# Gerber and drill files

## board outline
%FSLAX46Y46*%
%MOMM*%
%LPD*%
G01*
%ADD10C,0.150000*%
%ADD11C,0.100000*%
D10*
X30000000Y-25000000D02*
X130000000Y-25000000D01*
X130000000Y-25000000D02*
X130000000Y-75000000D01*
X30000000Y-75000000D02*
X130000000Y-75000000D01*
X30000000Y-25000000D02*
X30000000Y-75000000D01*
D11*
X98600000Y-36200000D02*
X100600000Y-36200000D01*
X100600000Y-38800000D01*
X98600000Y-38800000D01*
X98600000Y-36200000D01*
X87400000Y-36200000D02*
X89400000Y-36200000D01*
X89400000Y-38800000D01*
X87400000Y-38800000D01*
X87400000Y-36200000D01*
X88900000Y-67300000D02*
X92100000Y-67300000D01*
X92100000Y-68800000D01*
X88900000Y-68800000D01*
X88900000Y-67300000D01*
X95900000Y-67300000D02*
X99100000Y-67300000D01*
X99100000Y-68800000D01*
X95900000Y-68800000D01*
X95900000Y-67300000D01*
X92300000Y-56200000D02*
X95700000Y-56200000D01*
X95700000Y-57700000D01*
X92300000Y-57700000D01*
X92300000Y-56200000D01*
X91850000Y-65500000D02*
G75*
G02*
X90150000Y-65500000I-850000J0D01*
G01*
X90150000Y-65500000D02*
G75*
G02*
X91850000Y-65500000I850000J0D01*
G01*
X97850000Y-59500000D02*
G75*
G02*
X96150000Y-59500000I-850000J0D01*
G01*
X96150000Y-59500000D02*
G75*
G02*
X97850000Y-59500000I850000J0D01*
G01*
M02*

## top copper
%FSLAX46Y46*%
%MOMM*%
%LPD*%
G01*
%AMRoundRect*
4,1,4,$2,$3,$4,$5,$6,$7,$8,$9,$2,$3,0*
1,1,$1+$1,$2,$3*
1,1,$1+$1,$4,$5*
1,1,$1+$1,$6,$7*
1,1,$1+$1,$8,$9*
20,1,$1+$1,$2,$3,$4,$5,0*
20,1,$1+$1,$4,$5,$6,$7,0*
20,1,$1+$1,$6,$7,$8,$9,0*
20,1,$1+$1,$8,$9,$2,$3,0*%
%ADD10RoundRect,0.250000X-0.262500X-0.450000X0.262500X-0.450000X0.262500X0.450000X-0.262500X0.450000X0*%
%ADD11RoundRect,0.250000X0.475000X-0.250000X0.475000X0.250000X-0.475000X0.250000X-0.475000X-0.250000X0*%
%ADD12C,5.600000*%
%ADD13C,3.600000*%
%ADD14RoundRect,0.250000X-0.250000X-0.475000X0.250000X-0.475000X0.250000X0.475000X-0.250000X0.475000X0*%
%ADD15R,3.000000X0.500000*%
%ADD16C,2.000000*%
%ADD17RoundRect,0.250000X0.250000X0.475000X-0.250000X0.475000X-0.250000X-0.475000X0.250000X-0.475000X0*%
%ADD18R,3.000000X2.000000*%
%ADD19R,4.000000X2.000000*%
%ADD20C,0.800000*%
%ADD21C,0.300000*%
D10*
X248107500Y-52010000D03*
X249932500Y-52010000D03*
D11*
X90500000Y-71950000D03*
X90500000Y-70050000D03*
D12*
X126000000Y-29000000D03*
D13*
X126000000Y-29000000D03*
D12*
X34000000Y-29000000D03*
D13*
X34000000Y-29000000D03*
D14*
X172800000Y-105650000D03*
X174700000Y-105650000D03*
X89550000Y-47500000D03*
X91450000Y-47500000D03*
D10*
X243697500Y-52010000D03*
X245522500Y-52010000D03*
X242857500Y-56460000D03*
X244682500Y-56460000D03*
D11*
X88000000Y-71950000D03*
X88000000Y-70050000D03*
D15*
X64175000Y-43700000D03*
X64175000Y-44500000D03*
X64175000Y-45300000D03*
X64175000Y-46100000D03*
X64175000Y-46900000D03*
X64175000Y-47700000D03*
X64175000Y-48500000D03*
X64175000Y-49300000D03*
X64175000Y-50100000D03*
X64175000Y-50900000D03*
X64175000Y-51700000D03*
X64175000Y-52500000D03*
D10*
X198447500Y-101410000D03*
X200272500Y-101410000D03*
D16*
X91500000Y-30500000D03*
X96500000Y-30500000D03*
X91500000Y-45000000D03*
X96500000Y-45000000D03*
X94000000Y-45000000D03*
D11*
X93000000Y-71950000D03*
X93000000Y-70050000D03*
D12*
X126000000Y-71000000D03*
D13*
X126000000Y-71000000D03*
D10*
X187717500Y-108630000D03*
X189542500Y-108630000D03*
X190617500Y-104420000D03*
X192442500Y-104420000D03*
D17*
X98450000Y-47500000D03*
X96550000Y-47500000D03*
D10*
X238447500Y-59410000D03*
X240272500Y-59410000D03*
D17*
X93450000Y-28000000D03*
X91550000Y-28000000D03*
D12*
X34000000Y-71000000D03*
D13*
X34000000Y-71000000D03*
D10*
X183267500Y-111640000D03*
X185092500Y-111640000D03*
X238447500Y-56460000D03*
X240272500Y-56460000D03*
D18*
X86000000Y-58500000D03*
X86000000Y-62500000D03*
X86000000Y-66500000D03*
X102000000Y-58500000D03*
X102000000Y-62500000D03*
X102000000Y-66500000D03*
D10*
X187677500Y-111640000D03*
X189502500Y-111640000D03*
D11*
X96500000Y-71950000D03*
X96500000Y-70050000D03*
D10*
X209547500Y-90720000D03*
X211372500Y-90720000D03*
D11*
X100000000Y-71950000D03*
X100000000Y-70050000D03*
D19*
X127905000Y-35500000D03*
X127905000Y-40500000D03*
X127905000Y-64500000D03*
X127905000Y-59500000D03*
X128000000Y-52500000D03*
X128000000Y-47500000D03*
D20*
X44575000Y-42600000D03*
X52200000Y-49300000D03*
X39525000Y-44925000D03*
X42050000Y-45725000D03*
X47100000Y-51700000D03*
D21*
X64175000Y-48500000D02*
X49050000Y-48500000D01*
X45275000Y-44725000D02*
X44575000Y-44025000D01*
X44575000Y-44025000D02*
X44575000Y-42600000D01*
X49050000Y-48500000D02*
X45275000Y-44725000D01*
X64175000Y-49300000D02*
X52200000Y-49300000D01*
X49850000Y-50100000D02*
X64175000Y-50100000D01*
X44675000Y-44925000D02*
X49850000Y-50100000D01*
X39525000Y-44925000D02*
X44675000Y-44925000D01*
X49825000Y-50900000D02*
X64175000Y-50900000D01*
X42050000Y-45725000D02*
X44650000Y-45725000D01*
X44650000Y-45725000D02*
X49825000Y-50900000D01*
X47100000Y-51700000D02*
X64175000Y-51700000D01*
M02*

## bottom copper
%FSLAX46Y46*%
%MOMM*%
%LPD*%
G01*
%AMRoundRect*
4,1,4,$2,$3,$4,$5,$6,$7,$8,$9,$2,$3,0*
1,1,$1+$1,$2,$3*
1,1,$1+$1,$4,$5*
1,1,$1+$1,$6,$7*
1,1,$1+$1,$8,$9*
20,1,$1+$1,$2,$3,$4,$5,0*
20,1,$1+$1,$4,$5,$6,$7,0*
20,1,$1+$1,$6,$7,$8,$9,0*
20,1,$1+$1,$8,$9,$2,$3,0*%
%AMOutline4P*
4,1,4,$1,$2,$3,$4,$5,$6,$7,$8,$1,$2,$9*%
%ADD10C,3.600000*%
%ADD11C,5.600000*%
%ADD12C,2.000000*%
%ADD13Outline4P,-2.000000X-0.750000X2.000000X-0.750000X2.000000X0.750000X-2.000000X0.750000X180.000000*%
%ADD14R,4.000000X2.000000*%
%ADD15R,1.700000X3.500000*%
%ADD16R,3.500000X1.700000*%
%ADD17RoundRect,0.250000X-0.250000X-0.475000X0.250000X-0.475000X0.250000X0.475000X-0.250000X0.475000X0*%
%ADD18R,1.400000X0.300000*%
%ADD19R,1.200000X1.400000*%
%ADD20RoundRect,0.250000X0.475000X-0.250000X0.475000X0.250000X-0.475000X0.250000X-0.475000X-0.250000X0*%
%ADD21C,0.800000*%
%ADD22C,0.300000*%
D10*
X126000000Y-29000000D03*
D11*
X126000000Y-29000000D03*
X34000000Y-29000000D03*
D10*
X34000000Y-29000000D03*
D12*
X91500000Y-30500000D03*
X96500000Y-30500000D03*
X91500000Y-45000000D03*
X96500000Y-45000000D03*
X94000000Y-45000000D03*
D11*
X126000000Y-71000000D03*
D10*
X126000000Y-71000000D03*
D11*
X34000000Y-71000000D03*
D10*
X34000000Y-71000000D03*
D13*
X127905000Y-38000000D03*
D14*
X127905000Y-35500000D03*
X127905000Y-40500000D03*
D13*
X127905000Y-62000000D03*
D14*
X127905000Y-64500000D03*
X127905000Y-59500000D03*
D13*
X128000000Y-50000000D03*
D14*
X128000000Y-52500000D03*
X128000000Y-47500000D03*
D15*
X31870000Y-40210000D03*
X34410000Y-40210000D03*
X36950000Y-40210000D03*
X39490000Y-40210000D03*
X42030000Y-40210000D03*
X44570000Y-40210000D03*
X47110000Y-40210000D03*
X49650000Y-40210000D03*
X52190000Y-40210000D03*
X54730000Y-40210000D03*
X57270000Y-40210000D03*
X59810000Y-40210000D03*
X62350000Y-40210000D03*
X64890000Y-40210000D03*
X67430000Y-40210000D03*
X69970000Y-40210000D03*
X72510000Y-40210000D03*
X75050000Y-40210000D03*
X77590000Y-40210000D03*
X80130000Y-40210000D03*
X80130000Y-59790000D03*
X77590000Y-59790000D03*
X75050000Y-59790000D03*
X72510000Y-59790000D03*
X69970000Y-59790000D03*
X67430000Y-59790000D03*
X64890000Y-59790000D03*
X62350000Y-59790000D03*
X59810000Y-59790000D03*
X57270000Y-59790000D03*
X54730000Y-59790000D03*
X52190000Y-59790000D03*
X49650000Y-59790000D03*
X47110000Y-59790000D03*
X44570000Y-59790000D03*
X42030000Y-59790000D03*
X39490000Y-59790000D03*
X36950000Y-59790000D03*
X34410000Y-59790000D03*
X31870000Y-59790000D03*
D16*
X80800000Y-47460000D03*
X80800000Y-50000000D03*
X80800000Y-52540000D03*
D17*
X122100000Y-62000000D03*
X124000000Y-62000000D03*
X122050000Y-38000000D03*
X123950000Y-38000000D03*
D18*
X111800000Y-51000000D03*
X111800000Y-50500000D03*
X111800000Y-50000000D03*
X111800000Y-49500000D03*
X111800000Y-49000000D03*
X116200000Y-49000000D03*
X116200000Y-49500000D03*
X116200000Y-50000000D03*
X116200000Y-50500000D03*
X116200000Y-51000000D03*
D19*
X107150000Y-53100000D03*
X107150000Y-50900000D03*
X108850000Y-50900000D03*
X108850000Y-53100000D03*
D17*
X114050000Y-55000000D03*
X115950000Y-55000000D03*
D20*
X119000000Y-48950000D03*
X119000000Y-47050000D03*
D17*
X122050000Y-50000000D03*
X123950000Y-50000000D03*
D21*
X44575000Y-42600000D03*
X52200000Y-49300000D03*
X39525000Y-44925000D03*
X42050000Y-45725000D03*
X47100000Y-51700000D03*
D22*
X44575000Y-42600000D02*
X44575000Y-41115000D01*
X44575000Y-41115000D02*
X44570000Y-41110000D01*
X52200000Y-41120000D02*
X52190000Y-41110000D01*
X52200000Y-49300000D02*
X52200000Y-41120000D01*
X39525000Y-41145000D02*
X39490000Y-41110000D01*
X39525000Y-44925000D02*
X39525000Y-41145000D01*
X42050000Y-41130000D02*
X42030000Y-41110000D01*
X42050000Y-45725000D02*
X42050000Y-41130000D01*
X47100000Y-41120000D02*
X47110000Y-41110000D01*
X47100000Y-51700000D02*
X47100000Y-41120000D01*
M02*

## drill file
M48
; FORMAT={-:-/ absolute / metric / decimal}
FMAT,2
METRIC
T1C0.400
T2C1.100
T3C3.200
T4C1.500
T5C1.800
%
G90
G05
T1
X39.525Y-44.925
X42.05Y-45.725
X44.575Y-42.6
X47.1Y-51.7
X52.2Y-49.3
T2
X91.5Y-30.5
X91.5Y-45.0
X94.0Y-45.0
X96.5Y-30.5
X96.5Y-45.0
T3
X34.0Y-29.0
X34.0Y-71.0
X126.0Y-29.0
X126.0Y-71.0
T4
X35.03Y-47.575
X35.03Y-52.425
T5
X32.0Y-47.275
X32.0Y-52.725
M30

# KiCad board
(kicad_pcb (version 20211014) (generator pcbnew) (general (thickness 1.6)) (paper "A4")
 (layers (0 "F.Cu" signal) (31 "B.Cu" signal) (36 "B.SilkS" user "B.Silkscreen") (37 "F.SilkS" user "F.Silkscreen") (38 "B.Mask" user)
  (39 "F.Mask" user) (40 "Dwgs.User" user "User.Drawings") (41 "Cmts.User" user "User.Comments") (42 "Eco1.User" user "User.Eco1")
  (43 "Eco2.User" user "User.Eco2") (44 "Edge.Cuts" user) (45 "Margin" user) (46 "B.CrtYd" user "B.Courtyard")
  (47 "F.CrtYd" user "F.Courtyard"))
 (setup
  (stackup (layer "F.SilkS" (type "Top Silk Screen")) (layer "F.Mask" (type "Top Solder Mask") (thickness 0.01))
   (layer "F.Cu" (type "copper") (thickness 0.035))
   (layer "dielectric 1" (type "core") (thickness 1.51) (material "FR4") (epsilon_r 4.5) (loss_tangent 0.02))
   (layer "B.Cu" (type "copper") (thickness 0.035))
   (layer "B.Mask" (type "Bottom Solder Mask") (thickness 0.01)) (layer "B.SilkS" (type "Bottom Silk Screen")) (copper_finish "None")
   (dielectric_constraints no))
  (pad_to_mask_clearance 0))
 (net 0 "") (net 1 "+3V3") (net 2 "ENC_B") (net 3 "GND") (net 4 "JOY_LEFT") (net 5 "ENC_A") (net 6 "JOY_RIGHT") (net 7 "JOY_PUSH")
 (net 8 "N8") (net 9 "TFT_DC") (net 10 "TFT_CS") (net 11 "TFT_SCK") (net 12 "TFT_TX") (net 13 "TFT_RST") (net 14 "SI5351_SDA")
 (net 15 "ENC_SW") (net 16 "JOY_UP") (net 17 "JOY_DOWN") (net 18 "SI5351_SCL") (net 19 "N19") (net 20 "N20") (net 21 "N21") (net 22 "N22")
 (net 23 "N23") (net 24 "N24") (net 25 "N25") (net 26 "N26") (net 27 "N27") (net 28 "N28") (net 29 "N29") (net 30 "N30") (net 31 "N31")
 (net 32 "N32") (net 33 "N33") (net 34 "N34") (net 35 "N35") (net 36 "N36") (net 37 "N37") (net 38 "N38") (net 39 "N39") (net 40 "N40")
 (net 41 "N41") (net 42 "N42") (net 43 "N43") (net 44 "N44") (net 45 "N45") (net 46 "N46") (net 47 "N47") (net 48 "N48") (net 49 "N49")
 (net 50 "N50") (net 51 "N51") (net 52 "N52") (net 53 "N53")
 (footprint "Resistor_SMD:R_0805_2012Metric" (layer "F.Cu") (at 249.02 52.01)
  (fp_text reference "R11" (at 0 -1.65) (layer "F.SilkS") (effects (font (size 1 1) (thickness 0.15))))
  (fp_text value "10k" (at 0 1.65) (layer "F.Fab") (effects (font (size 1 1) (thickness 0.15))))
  (pad "1" smd roundrect (at -0.9125 0) (size 1.025 1.4) (layers "F.Cu" "F.Paste" "F.Mask") (roundrect_rratio 0.243902) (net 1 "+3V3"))
  (pad "2" smd roundrect (at 0.9125 0) (size 1.025 1.4) (layers "F.Cu" "F.Paste" "F.Mask") (roundrect_rratio 0.243902) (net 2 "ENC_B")))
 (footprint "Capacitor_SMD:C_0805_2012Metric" (layer "F.Cu") (at 90.5 71 90)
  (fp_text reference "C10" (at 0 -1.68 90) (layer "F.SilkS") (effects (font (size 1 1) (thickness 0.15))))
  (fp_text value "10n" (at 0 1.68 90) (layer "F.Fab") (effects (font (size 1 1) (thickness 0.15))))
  (pad "1" smd roundrect (at -0.95 0 90) (size 1 1.45) (layers "F.Cu" "F.Paste" "F.Mask") (roundrect_rratio 0.25) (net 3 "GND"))
  (pad "2" smd roundrect (at 0.95 0 90) (size 1 1.45) (layers "F.Cu" "F.Paste" "F.Mask") (roundrect_rratio 0.25) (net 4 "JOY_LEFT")))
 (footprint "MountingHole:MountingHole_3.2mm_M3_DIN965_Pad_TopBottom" (layer "F.Cu") (at 126 29)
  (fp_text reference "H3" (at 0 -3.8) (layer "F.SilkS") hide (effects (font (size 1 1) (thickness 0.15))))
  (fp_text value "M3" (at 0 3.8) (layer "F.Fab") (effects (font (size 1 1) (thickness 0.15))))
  (pad "1" connect circle (at 0 0) (size 5.6 5.6) (layers "F.Cu" "F.Mask"))
  (pad "1" thru_hole circle (at 0 0) (size 3.6 3.6) (drill 3.2) (layers *.Cu *.Mask))
  (pad "1" connect circle (at 0 0) (size 5.6 5.6) (layers "B.Cu" "B.Mask")))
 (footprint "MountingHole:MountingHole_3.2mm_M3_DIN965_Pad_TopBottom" (layer "F.Cu") (at 34 29)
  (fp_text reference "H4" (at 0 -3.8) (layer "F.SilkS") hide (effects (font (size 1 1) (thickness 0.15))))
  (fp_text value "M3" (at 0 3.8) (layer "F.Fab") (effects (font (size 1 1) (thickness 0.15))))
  (pad "1" connect circle (at 0 0) (size 5.6 5.6) (layers "F.Cu" "F.Mask"))
  (pad "1" connect circle (at 0 0) (size 5.6 5.6) (layers "B.Cu" "B.Mask"))
  (pad "1" thru_hole circle (at 0 0) (size 3.6 3.6) (drill 3.2) (layers *.Cu *.Mask)))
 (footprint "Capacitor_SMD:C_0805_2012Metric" (layer "F.Cu") (at 173.75 105.65)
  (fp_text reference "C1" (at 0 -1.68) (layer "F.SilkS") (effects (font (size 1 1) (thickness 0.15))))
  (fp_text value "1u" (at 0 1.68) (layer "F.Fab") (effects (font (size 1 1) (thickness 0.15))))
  (pad "1" smd roundrect (at -0.95 0) (size 1 1.45) (layers "F.Cu" "F.Paste" "F.Mask") (roundrect_rratio 0.25) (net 1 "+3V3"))
  (pad "2" smd roundrect (at 0.95 0) (size 1 1.45) (layers "F.Cu" "F.Paste" "F.Mask") (roundrect_rratio 0.25) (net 3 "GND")))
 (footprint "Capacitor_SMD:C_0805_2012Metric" (layer "F.Cu") (at 90.5 47.5)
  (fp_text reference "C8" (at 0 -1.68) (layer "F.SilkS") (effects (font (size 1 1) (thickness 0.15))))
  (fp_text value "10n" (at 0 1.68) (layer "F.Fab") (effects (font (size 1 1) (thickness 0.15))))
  (pad "1" smd roundrect (at -0.95 0) (size 1 1.45) (layers "F.Cu" "F.Paste" "F.Mask") (roundrect_rratio 0.25) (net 3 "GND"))
  (pad "2" smd roundrect (at 0.95 0) (size 1 1.45) (layers "F.Cu" "F.Paste" "F.Mask") (roundrect_rratio 0.25) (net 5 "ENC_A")))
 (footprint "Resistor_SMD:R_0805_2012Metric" (layer "F.Cu") (at 244.61 52.01)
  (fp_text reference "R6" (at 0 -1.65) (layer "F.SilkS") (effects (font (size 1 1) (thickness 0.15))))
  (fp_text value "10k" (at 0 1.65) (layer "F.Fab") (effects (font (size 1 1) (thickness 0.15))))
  (pad "1" smd roundrect (at -0.9125 0) (size 1.025 1.4) (layers "F.Cu" "F.Paste" "F.Mask") (roundrect_rratio 0.243902) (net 1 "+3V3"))
  (pad "2" smd roundrect (at 0.9125 0) (size 1.025 1.4) (layers "F.Cu" "F.Paste" "F.Mask") (roundrect_rratio 0.243902) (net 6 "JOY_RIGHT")))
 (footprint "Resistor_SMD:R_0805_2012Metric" (layer "F.Cu") (at 243.77 56.46)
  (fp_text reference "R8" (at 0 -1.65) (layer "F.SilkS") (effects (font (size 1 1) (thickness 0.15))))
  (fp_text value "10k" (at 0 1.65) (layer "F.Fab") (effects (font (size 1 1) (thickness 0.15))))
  (pad "1" smd roundrect (at -0.9125 0) (size 1.025 1.4) (layers "F.Cu" "F.Paste" "F.Mask") (roundrect_rratio 0.243902) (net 1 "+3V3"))
  (pad "2" smd roundrect (at 0.9125 0) (size 1.025 1.4) (layers "F.Cu" "F.Paste" "F.Mask") (roundrect_rratio 0.243902) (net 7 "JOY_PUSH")))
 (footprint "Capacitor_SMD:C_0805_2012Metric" (layer "F.Cu") (at 88 71 90)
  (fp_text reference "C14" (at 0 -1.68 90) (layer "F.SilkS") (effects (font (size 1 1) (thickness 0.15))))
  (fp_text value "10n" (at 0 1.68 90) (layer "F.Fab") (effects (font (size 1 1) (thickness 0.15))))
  (pad "1" smd roundrect (at -0.95 0 90) (size 1 1.45) (layers "F.Cu" "F.Paste" "F.Mask") (roundrect_rratio 0.25) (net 3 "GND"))
  (pad "2" smd roundrect (at 0.95 0 90) (size 1 1.45) (layers "F.Cu" "F.Paste" "F.Mask") (roundrect_rratio 0.25) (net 7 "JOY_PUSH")))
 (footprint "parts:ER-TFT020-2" (layer "F.Cu") (at 58 50)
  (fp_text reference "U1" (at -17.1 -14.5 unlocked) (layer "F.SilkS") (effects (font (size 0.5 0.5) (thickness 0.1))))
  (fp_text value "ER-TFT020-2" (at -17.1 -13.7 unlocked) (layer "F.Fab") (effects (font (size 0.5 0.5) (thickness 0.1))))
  (pad "1" smd rect (at 6.175 -6.3) (size 3 0.5) (layers "F.Cu" "B.Paste" "B.Mask") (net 3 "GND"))
  (pad "2" smd rect (at 6.175 -5.5) (size 3 0.5) (layers "F.Cu" "B.Paste" "B.Mask") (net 3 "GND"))
  (pad "3" smd rect (at 6.175 -4.7) (size 3 0.5) (layers "F.Cu" "B.Paste" "B.Mask") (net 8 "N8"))
  (pad "4" smd rect (at 6.175 -3.9) (size 3 0.5) (layers "F.Cu" "B.Paste" "B.Mask") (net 1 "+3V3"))
  (pad "5" smd rect (at 6.175 -3.1) (size 3 0.5) (layers "F.Cu" "B.Paste" "B.Mask") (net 3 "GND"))
  (pad "6" smd rect (at 6.175 -2.3) (size 3 0.5) (layers "F.Cu" "B.Paste" "B.Mask") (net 3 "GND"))
  (pad "7" smd rect (at 6.175 -1.5) (size 3 0.5) (layers "F.Cu" "B.Paste" "B.Mask") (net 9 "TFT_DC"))
  (pad "8" smd rect (at 6.175 -0.7) (size 3 0.5) (layers "F.Cu" "B.Paste" "B.Mask") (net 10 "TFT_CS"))
  (pad "9" smd rect (at 6.175 0.1) (size 3 0.5) (layers "F.Cu" "B.Paste" "B.Mask") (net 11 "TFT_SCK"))
  (pad "10" smd rect (at 6.175 0.9) (size 3 0.5) (layers "F.Cu" "B.Paste" "B.Mask") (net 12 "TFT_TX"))
  (pad "11" smd rect (at 6.175 1.7) (size 3 0.5) (layers "F.Cu" "B.Paste" "B.Mask") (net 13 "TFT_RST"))
  (pad "12" smd rect (at 6.175 2.5) (size 3 0.5) (layers "F.Cu" "B.Paste" "B.Mask") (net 3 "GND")))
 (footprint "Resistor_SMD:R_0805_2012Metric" (layer "F.Cu") (at 199.36 101.41)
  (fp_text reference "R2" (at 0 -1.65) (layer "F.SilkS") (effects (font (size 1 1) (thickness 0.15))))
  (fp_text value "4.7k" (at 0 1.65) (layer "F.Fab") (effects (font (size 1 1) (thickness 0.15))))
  (pad "1" smd roundrect (at -0.9125 0) (size 1.025 1.4) (layers "F.Cu" "F.Paste" "F.Mask") (roundrect_rratio 0.243902)
   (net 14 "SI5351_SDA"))
  (pad "2" smd roundrect (at 0.9125 0) (size 1.025 1.4) (layers "F.Cu" "F.Paste" "F.Mask") (roundrect_rratio 0.243902) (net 1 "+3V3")))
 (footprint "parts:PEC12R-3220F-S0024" (layer "F.Cu") (at 94 37.5)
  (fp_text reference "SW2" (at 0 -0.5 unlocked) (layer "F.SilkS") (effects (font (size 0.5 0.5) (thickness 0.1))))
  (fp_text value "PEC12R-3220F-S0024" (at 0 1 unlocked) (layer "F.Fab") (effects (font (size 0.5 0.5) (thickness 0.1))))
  (fp_rect (start 4.6 -1.3) (end 6.6 1.3) (layer "Edge.Cuts") (width 0.1) (fill none))
  (fp_rect (start -6.6 -1.3) (end -4.6 1.3) (layer "Edge.Cuts") (width 0.1) (fill none))
  (pad "1" thru_hole circle (at -2.5 -7) (size 2 2) (drill 1.1) (layers *.Cu *.Mask) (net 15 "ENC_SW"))
  (pad "2" thru_hole circle (at 2.5 -7) (size 2 2) (drill 1.1) (layers *.Cu *.Mask) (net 3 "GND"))
  (pad "A" thru_hole circle (at -2.5 7.5) (size 2 2) (drill 1.1) (layers *.Cu *.Mask) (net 5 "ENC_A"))
  (pad "B" thru_hole circle (at 2.5 7.5) (size 2 2) (drill 1.1) (layers *.Cu *.Mask) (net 2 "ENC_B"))
  (pad "C" thru_hole circle (at 0 7.5) (size 2 2) (drill 1.1) (layers *.Cu *.Mask) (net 3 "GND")))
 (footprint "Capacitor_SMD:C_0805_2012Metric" (layer "F.Cu") (at 93 71 90)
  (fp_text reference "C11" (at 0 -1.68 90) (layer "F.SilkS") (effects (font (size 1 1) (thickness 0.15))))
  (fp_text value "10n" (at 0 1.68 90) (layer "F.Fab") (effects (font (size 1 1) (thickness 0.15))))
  (pad "1" smd roundrect (at -0.95 0 90) (size 1 1.45) (layers "F.Cu" "F.Paste" "F.Mask") (roundrect_rratio 0.25) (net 3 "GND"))
  (pad "2" smd roundrect (at 0.95 0 90) (size 1 1.45) (layers "F.Cu" "F.Paste" "F.Mask") (roundrect_rratio 0.25) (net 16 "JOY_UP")))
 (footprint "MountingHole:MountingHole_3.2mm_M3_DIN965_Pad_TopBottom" (layer "F.Cu") (at 126 71)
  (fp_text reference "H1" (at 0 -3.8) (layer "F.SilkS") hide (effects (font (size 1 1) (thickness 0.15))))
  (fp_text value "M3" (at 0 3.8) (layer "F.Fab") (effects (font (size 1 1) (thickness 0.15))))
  (pad "1" connect circle (at 0 0) (size 5.6 5.6) (layers "B.Cu" "B.Mask"))
  (pad "1" connect circle (at 0 0) (size 5.6 5.6) (layers "F.Cu" "F.Mask"))
  (pad "1" thru_hole circle (at 0 0) (size 3.6 3.6) (drill 3.2) (layers *.Cu *.Mask)))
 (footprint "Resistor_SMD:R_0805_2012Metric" (layer "F.Cu") (at 188.63 108.63)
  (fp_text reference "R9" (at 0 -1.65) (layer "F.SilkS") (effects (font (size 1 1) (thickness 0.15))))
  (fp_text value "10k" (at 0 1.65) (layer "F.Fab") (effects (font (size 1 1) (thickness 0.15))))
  (pad "1" smd roundrect (at -0.9125 0) (size 1.025 1.4) (layers "F.Cu" "F.Paste" "F.Mask") (roundrect_rratio 0.243902) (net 1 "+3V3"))
  (pad "2" smd roundrect (at 0.9125 0) (size 1.025 1.4) (layers "F.Cu" "F.Paste" "F.Mask") (roundrect_rratio 0.243902) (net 15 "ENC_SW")))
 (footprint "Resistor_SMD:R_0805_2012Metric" (layer "F.Cu") (at 191.53 104.42)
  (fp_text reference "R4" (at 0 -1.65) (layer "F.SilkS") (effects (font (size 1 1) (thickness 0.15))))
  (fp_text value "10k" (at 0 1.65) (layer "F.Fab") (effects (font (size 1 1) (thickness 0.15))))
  (pad "1" smd roundrect (at -0.9125 0) (size 1.025 1.4) (layers "F.Cu" "F.Paste" "F.Mask") (roundrect_rratio 0.243902) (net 1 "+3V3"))
  (pad "2" smd roundrect (at 0.9125 0) (size 1.025 1.4) (layers "F.Cu" "F.Paste" "F.Mask") (roundrect_rratio 0.243902) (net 4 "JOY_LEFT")))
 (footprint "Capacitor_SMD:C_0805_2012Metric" (layer "F.Cu") (at 97.5 47.5 180)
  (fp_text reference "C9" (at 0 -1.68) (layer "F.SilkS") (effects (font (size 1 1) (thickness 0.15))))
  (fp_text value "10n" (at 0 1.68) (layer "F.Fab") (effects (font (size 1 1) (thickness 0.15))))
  (pad "1" smd roundrect (at -0.95 0 180) (size 1 1.45) (layers "F.Cu" "F.Paste" "F.Mask") (roundrect_rratio 0.25) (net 3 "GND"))
  (pad "2" smd roundrect (at 0.95 0 180) (size 1 1.45) (layers "F.Cu" "F.Paste" "F.Mask") (roundrect_rratio 0.25) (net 2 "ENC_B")))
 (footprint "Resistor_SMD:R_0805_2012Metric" (layer "F.Cu") (at 239.36 59.41)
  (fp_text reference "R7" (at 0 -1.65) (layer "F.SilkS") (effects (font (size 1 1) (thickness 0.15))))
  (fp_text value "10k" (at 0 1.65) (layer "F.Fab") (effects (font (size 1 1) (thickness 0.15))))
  (pad "1" smd roundrect (at -0.9125 0) (size 1.025 1.4) (layers "F.Cu" "F.Paste" "F.Mask") (roundrect_rratio 0.243902) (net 1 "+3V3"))
  (pad "2" smd roundrect (at 0.9125 0) (size 1.025 1.4) (layers "F.Cu" "F.Paste" "F.Mask") (roundrect_rratio 0.243902) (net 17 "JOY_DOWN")))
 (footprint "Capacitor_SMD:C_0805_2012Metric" (layer "F.Cu") (at 92.5 28 180)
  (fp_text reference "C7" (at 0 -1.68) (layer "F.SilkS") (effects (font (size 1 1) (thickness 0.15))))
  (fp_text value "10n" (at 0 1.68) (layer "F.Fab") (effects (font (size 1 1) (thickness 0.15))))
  (pad "1" smd roundrect (at -0.95 0 180) (size 1 1.45) (layers "F.Cu" "F.Paste" "F.Mask") (roundrect_rratio 0.25) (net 3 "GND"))
  (pad "2" smd roundrect (at 0.95 0 180) (size 1 1.45) (layers "F.Cu" "F.Paste" "F.Mask") (roundrect_rratio 0.25) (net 15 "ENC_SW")))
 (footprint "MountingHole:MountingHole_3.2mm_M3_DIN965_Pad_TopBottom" (layer "F.Cu") (at 34 71)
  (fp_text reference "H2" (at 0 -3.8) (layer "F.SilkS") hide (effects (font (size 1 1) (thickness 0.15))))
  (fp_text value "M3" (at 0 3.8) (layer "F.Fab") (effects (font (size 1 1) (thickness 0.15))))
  (pad "1" connect circle (at 0 0) (size 5.6 5.6) (layers "B.Cu" "B.Mask"))
  (pad "1" connect circle (at 0 0) (size 5.6 5.6) (layers "F.Cu" "F.Mask"))
  (pad "1" thru_hole circle (at 0 0) (size 3.6 3.6) (drill 3.2) (layers *.Cu *.Mask)))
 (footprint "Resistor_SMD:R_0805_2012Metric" (layer "F.Cu") (at 184.18 111.64)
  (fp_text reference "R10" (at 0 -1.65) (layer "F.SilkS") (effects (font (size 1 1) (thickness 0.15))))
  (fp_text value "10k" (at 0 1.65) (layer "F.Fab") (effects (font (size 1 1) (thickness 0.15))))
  (pad "1" smd roundrect (at -0.9125 0) (size 1.025 1.4) (layers "F.Cu" "F.Paste" "F.Mask") (roundrect_rratio 0.243902) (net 1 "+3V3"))
  (pad "2" smd roundrect (at 0.9125 0) (size 1.025 1.4) (layers "F.Cu" "F.Paste" "F.Mask") (roundrect_rratio 0.243902) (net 5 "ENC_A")))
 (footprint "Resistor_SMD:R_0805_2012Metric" (layer "F.Cu") (at 239.36 56.46)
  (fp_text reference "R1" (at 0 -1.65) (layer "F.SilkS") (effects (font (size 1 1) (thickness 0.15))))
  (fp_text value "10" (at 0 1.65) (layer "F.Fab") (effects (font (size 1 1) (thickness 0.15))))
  (pad "1" smd roundrect (at -0.9125 0) (size 1.025 1.4) (layers "F.Cu" "F.Paste" "F.Mask") (roundrect_rratio 0.243902) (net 8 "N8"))
  (pad "2" smd roundrect (at 0.9125 0) (size 1.025 1.4) (layers "F.Cu" "F.Paste" "F.Mask") (roundrect_rratio 0.243902) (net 1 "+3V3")))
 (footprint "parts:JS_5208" (layer "F.Cu") (at 94 62.5)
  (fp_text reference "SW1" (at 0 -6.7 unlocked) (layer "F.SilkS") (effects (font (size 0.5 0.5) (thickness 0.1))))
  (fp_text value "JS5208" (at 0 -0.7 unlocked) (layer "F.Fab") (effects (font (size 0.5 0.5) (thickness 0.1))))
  (fp_rect (start -5.1 4.8) (end -1.9 6.3) (layer "Edge.Cuts") (width 0.1) (fill none))
  (fp_rect (start 1.9 4.8) (end 5.1 6.3) (layer "Edge.Cuts") (width 0.1) (fill none))
  (fp_rect (start -1.7 -6.3) (end 1.7 -4.8) (layer "Edge.Cuts") (width 0.1) (fill none))
  (fp_circle (center -3 3) (end -2.15 3) (layer "Edge.Cuts") (width 0.1) (fill none))
  (fp_circle (center 3 -3) (end 3.85 -3) (layer "Edge.Cuts") (width 0.1) (fill none))
  (pad "1" smd rect (at -8 -4) (size 3 2) (layers "F.Cu" "F.Paste" "F.Mask") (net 3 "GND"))
  (pad "2" smd rect (at -8 0) (size 3 2) (layers "F.Cu" "F.Paste" "F.Mask") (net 4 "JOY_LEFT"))
  (pad "3" smd rect (at -8 4) (size 3 2) (layers "F.Cu" "F.Paste" "F.Mask") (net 7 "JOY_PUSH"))
  (pad "4" smd rect (at 8 -4) (size 3 2) (layers "F.Cu" "F.Paste" "F.Mask") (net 16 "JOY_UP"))
  (pad "5" smd rect (at 8 0) (size 3 2) (layers "F.Cu" "F.Paste" "F.Mask") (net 6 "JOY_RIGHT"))
  (pad "6" smd rect (at 8 4) (size 3 2) (layers "F.Cu" "F.Paste" "F.Mask") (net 17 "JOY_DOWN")))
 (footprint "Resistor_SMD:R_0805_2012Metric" (layer "F.Cu") (at 188.59 111.64)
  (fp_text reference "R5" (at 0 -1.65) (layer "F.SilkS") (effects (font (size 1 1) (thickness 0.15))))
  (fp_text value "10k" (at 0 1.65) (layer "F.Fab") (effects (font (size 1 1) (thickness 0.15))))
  (pad "1" smd roundrect (at -0.9125 0) (size 1.025 1.4) (layers "F.Cu" "F.Paste" "F.Mask") (roundrect_rratio 0.243902) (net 1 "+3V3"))
  (pad "2" smd roundrect (at 0.9125 0) (size 1.025 1.4) (layers "F.Cu" "F.Paste" "F.Mask") (roundrect_rratio 0.243902) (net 16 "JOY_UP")))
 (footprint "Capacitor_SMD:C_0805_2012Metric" (layer "F.Cu") (at 96.5 71 90)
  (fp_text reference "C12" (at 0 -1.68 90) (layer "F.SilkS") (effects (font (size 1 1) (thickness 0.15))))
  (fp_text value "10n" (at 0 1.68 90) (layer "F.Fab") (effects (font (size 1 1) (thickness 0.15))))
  (pad "1" smd roundrect (at -0.95 0 90) (size 1 1.45) (layers "F.Cu" "F.Paste" "F.Mask") (roundrect_rratio 0.25) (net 3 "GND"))
  (pad "2" smd roundrect (at 0.95 0 90) (size 1 1.45) (layers "F.Cu" "F.Paste" "F.Mask") (roundrect_rratio 0.25) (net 6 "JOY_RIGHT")))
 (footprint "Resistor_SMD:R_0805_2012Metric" (layer "F.Cu") (at 210.46 90.72)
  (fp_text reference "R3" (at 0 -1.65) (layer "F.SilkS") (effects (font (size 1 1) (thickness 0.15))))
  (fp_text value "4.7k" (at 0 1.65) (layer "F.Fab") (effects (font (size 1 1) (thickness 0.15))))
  (pad "1" smd roundrect (at -0.9125 0) (size 1.025 1.4) (layers "F.Cu" "F.Paste" "F.Mask") (roundrect_rratio 0.243902)
   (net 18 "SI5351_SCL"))
  (pad "2" smd roundrect (at 0.9125 0) (size 1.025 1.4) (layers "F.Cu" "F.Paste" "F.Mask") (roundrect_rratio 0.243902) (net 1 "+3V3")))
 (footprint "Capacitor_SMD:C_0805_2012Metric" (layer "F.Cu") (at 100 71 90)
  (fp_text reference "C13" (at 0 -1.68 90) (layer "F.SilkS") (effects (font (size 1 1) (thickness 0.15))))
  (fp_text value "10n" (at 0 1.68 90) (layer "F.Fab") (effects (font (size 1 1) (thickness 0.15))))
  (pad "1" smd roundrect (at -0.95 0 90) (size 1 1.45) (layers "F.Cu" "F.Paste" "F.Mask") (roundrect_rratio 0.25) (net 3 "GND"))
  (pad "2" smd roundrect (at 0.95 0 90) (size 1 1.45) (layers "F.Cu" "F.Paste" "F.Mask") (roundrect_rratio 0.25) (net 17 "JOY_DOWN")))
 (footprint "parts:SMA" (layer "B.Cu") (at 129.905 38 180)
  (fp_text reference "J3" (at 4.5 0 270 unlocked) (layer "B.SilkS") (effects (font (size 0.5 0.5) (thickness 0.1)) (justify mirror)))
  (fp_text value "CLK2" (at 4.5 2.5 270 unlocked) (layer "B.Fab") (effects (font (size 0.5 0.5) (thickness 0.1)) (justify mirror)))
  (pad "1" smd trapezoid (at 2 0 180) (size 4 1.5) (layers "B.Cu" "B.Paste" "B.Mask") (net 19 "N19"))
  (pad "2" smd rect (at 2 2.5 180) (size 4 2) (layers "B.Cu" "B.Paste" "B.Mask") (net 3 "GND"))
  (pad "2" smd rect (at 2 2.5 180) (size 4 2) (layers "F.Cu" "B.Paste" "B.Mask") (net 3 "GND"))
  (pad "2" smd rect (at 2 -2.5 180) (size 4 2) (layers "B.Cu" "B.Paste" "B.Mask") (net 3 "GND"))
  (pad "2" smd rect (at 2 -2.5 180) (size 4 2) (layers "F.Cu" "B.Paste" "B.Mask") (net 3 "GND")))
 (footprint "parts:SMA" (layer "B.Cu") (at 129.905 62 180)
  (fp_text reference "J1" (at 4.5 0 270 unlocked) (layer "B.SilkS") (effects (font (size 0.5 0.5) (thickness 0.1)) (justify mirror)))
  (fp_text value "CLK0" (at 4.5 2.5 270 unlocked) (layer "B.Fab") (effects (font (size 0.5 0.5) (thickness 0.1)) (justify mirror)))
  (pad "1" smd trapezoid (at 2 0 180) (size 4 1.5) (layers "B.Cu" "B.Paste" "B.Mask") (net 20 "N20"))
  (pad "2" smd rect (at 2 -2.5 180) (size 4 2) (layers "B.Cu" "B.Paste" "B.Mask") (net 3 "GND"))
  (pad "2" smd rect (at 2 -2.5 180) (size 4 2) (layers "F.Cu" "B.Paste" "B.Mask") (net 3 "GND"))
  (pad "2" smd rect (at 2 2.5 180) (size 4 2) (layers "B.Cu" "B.Paste" "B.Mask") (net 3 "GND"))
  (pad "2" smd rect (at 2 2.5 180) (size 4 2) (layers "F.Cu" "B.Paste" "B.Mask") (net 3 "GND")))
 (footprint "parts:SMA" (layer "B.Cu") (at 130 50 180)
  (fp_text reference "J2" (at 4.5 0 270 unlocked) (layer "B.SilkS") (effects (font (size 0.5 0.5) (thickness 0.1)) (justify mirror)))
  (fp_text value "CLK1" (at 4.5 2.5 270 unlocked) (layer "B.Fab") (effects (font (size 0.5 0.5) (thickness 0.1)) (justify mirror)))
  (pad "1" smd trapezoid (at 2 0 180) (size 4 1.5) (layers "B.Cu" "B.Paste" "B.Mask") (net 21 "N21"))
  (pad "2" smd rect (at 2 -2.5 180) (size 4 2) (layers "B.Cu" "B.Paste" "B.Mask") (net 3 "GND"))
  (pad "2" smd rect (at 2 2.5 180) (size 4 2) (layers "B.Cu" "B.Paste" "B.Mask") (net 3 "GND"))
  (pad "2" smd rect (at 2 -2.5 180) (size 4 2) (layers "F.Cu" "B.Paste" "B.Mask") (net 3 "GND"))
  (pad "2" smd rect (at 2 2.5 180) (size 4 2) (layers "F.Cu" "B.Paste" "B.Mask") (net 3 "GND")))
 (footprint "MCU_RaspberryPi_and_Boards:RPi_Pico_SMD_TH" (layer "B.Cu") (at 56 50 -90)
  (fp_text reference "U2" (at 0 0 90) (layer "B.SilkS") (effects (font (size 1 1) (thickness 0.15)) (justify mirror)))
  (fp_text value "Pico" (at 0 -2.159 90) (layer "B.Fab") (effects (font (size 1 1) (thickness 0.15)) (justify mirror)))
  (pad "" np_thru_hole oval (at 2.425 20.97 270) (size 1.5 1.5) (drill 1.5) (layers *.Cu *.Mask))
  (pad "" np_thru_hole oval (at 2.725 24 270) (size 1.8 1.8) (drill 1.8) (layers *.Cu *.Mask))
  (pad "" np_thru_hole oval (at -2.725 24 270) (size 1.8 1.8) (drill 1.8) (layers *.Cu *.Mask))
  (pad "" np_thru_hole oval (at -2.425 20.97 270) (size 1.5 1.5) (drill 1.5) (layers *.Cu *.Mask))
  (pad "1" smd rect (at -8.89 24.13 270) (size 3.5 1.7) (drill (offset -0.9 0)) (layers "B.Cu" "B.Mask") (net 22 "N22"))
  (pad "2" smd rect (at -8.89 21.59 270) (size 3.5 1.7) (drill (offset -0.9 0)) (layers "B.Cu" "B.Mask") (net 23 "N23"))
  (pad "3" smd rect (at -8.89 19.05 270) (size 3.5 1.7) (drill (offset -0.9 0)) (layers "B.Cu" "B.Mask") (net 3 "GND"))
  (pad "4" smd rect (at -8.89 16.51 270) (size 3.5 1.7) (drill (offset -0.9 0)) (layers "B.Cu" "B.Mask") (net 11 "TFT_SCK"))
  (pad "5" smd rect (at -8.89 13.97 270) (size 3.5 1.7) (drill (offset -0.9 0)) (layers "B.Cu" "B.Mask") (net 12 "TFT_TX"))
  (pad "6" smd rect (at -8.89 11.43 270) (size 3.5 1.7) (drill (offset -0.9 0)) (layers "B.Cu" "B.Mask") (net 9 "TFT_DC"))
  (pad "7" smd rect (at -8.89 8.89 270) (size 3.5 1.7) (drill (offset -0.9 0)) (layers "B.Cu" "B.Mask") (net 13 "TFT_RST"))
  (pad "8" smd rect (at -8.89 6.35 270) (size 3.5 1.7) (drill (offset -0.9 0)) (layers "B.Cu" "B.Mask") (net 3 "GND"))
  (pad "9" smd rect (at -8.89 3.81 270) (size 3.5 1.7) (drill (offset -0.9 0)) (layers "B.Cu" "B.Mask") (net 10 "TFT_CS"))
  (pad "10" smd rect (at -8.89 1.27 270) (size 3.5 1.7) (drill (offset -0.9 0)) (layers "B.Cu" "B.Mask") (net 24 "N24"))
  (pad "11" smd rect (at -8.89 -1.27 270) (size 3.5 1.7) (drill (offset -0.9 0)) (layers "B.Cu" "B.Mask") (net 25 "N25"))
  (pad "12" smd rect (at -8.89 -3.81 270) (size 3.5 1.7) (drill (offset -0.9 0)) (layers "B.Cu" "B.Mask") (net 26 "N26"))
  (pad "13" smd rect (at -8.89 -6.35 270) (size 3.5 1.7) (drill (offset -0.9 0)) (layers "B.Cu" "B.Mask") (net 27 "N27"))
  (pad "14" smd rect (at -8.89 -8.89 270) (size 3.5 1.7) (drill (offset -0.9 0)) (layers "B.Cu" "B.Mask") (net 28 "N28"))
  (pad "15" smd rect (at -8.89 -11.43 270) (size 3.5 1.7) (drill (offset -0.9 0)) (layers "B.Cu" "B.Mask") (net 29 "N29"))
  (pad "16" smd rect (at -8.89 -13.97 270) (size 3.5 1.7) (drill (offset -0.9 0)) (layers "B.Cu" "B.Mask") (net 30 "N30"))
  (pad "17" smd rect (at -8.89 -16.51 270) (size 3.5 1.7) (drill (offset -0.9 0)) (layers "B.Cu" "B.Mask") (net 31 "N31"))
  (pad "18" smd rect (at -8.89 -19.05 270) (size 3.5 1.7) (drill (offset -0.9 0)) (layers "B.Cu" "B.Mask") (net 3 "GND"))
  (pad "19" smd rect (at -8.89 -21.59 270) (size 3.5 1.7) (drill (offset -0.9 0)) (layers "B.Cu" "B.Mask") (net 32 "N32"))
  (pad "20" smd rect (at -8.89 -24.13 270) (size 3.5 1.7) (drill (offset -0.9 0)) (layers "B.Cu" "B.Mask") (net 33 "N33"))
  (pad "21" smd rect (at 8.89 -24.13 270) (size 3.5 1.7) (drill (offset 0.9 0)) (layers "B.Cu" "B.Mask") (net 14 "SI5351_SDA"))
  (pad "22" smd rect (at 8.89 -21.59 270) (size 3.5 1.7) (drill (offset 0.9 0)) (layers "B.Cu" "B.Mask") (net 18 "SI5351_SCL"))
  (pad "23" smd rect (at 8.89 -19.05 270) (size 3.5 1.7) (drill (offset 0.9 0)) (layers "B.Cu" "B.Mask") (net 3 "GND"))
  (pad "24" smd rect (at 8.89 -16.51 270) (size 3.5 1.7) (drill (offset 0.9 0)) (layers "B.Cu" "B.Mask") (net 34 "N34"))
  (pad "25" smd rect (at 8.89 -13.97 270) (size 3.5 1.7) (drill (offset 0.9 0)) (layers "B.Cu" "B.Mask") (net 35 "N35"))
  (pad "26" smd rect (at 8.89 -11.43 270) (size 3.5 1.7) (drill (offset 0.9 0)) (layers "B.Cu" "B.Mask") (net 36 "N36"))
  (pad "27" smd rect (at 8.89 -8.89 270) (size 3.5 1.7) (drill (offset 0.9 0)) (layers "B.Cu" "B.Mask") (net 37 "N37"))
  (pad "28" smd rect (at 8.89 -6.35 270) (size 3.5 1.7) (drill (offset 0.9 0)) (layers "B.Cu" "B.Mask") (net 3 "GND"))
  (pad "29" smd rect (at 8.89 -3.81 270) (size 3.5 1.7) (drill (offset 0.9 0)) (layers "B.Cu" "B.Mask") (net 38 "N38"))
  (pad "30" smd rect (at 8.89 -1.27 270) (size 3.5 1.7) (drill (offset 0.9 0)) (layers "B.Cu" "B.Mask") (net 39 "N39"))
  (pad "31" smd rect (at 8.89 1.27 270) (size 3.5 1.7) (drill (offset 0.9 0)) (layers "B.Cu" "B.Mask") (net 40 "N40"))
  (pad "32" smd rect (at 8.89 3.81 270) (size 3.5 1.7) (drill (offset 0.9 0)) (layers "B.Cu" "B.Mask") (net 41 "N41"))
  (pad "33" smd rect (at 8.89 6.35 270) (size 3.5 1.7) (drill (offset 0.9 0)) (layers "B.Cu" "B.Mask") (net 3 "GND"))
  (pad "34" smd rect (at 8.89 8.89 270) (size 3.5 1.7) (drill (offset 0.9 0)) (layers "B.Cu" "B.Mask") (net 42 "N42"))
  (pad "35" smd rect (at 8.89 11.43 270) (size 3.5 1.7) (drill (offset 0.9 0)) (layers "B.Cu" "B.Mask") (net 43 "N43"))
  (pad "36" smd rect (at 8.89 13.97 270) (size 3.5 1.7) (drill (offset 0.9 0)) (layers "B.Cu" "B.Mask") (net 1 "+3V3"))
  (pad "37" smd rect (at 8.89 16.51 270) (size 3.5 1.7) (drill (offset 0.9 0)) (layers "B.Cu" "B.Mask") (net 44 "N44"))
  (pad "38" smd rect (at 8.89 19.05 270) (size 3.5 1.7) (drill (offset 0.9 0)) (layers "B.Cu" "B.Mask") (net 3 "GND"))
  (pad "39" smd rect (at 8.89 21.59 270) (size 3.5 1.7) (drill (offset 0.9 0)) (layers "B.Cu" "B.Mask") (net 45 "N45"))
  (pad "40" smd rect (at 8.89 24.13 270) (size 3.5 1.7) (drill (offset 0.9 0)) (layers "B.Cu" "B.Mask") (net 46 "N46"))
  (pad "41" smd rect (at -2.54 -23.9 180) (size 3.5 1.7) (drill (offset -0.9 0)) (layers "B.Cu" "B.Mask") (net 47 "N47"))
  (pad "42" smd rect (at 0 -23.9 180) (size 3.5 1.7) (drill (offset -0.9 0)) (layers "B.Cu" "B.Mask") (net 3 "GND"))
  (pad "43" smd rect (at 2.54 -23.9 180) (size 3.5 1.7) (drill (offset -0.9 0)) (layers "B.Cu" "B.Mask") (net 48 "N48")))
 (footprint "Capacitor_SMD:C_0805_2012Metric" (layer "B.Cu") (at 123.05 62)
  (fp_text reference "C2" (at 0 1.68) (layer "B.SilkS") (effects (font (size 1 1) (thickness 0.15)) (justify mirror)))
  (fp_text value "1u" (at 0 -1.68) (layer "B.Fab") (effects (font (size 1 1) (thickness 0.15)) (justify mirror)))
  (pad "1" smd roundrect (at -0.95 0) (size 1 1.45) (layers "B.Cu" "B.Paste" "B.Mask") (roundrect_rratio 0.25) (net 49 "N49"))
  (pad "2" smd roundrect (at 0.95 0) (size 1 1.45) (layers "B.Cu" "B.Paste" "B.Mask") (roundrect_rratio 0.25) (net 20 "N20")))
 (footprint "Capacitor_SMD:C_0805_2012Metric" (layer "B.Cu") (at 123 38)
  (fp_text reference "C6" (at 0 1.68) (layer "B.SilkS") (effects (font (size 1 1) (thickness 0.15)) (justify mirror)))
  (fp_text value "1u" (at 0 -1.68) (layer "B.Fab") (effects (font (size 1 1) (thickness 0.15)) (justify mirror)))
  (pad "1" smd roundrect (at -0.95 0) (size 1 1.45) (layers "B.Cu" "B.Paste" "B.Mask") (roundrect_rratio 0.25) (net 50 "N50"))
  (pad "2" smd roundrect (at 0.95 0) (size 1 1.45) (layers "B.Cu" "B.Paste" "B.Mask") (roundrect_rratio 0.25) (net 19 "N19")))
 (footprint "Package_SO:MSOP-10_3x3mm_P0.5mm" (layer "B.Cu") (at 114 50)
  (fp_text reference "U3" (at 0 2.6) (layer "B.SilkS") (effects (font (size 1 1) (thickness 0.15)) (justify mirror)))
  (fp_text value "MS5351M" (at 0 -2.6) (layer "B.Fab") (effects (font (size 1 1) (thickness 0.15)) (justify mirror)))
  (pad "1" smd rect (at -2.2 1) (size 1.4 0.3) (layers "B.Cu" "B.Paste" "B.Mask") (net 1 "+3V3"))
  (pad "2" smd rect (at -2.2 0.5) (size 1.4 0.3) (layers "B.Cu" "B.Paste" "B.Mask") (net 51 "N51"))
  (pad "3" smd rect (at -2.2 0) (size 1.4 0.3) (layers "B.Cu" "B.Paste" "B.Mask") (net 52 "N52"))
  (pad "4" smd rect (at -2.2 -0.5) (size 1.4 0.3) (layers "B.Cu" "B.Paste" "B.Mask") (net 18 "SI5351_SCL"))
  (pad "5" smd rect (at -2.2 -1) (size 1.4 0.3) (layers "B.Cu" "B.Paste" "B.Mask") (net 14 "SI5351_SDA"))
  (pad "6" smd rect (at 2.2 -1) (size 1.4 0.3) (layers "B.Cu" "B.Paste" "B.Mask") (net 50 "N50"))
  (pad "7" smd rect (at 2.2 -0.5) (size 1.4 0.3) (layers "B.Cu" "B.Paste" "B.Mask") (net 1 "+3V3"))
  (pad "8" smd rect (at 2.2 0) (size 1.4 0.3) (layers "B.Cu" "B.Paste" "B.Mask") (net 3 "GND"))
  (pad "9" smd rect (at 2.2 0.5) (size 1.4 0.3) (layers "B.Cu" "B.Paste" "B.Mask") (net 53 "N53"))
  (pad "10" smd rect (at 2.2 1) (size 1.4 0.3) (layers "B.Cu" "B.Paste" "B.Mask") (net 49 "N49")))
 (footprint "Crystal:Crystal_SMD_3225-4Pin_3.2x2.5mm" (layer "B.Cu") (at 108 52 90)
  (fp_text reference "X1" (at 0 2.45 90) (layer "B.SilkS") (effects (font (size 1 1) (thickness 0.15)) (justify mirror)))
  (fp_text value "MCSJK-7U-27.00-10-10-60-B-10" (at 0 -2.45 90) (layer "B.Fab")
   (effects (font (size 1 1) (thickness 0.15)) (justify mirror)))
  (pad "1" smd rect (at -1.1 -0.85 90) (size 1.4 1.2) (layers "B.Cu" "B.Paste" "B.Mask") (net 51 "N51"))
  (pad "2" smd rect (at 1.1 -0.85 90) (size 1.4 1.2) (layers "B.Cu" "B.Paste" "B.Mask") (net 3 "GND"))
  (pad "3" smd rect (at 1.1 0.85 90) (size 1.4 1.2) (layers "B.Cu" "B.Paste" "B.Mask") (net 52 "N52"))
  (pad "4" smd rect (at -1.1 0.85 90) (size 1.4 1.2) (layers "B.Cu" "B.Paste" "B.Mask") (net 3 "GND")))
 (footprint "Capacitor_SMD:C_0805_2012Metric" (layer "B.Cu") (at 115 55)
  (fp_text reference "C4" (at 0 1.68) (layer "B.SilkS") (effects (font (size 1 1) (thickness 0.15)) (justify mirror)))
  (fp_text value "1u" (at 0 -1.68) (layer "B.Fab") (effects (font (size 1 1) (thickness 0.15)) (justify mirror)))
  (pad "1" smd roundrect (at -0.95 0) (size 1 1.45) (layers "B.Cu" "B.Paste" "B.Mask") (roundrect_rratio 0.25) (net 1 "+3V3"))
  (pad "2" smd roundrect (at 0.95 0) (size 1 1.45) (layers "B.Cu" "B.Paste" "B.Mask") (roundrect_rratio 0.25) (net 3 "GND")))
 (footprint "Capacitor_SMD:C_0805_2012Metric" (layer "B.Cu") (at 119 48 90)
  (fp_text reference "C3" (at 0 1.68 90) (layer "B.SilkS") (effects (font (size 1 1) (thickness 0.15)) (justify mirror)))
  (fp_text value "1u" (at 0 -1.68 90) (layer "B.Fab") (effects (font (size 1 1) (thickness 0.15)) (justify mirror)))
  (pad "1" smd roundrect (at -0.95 0 90) (size 1 1.45) (layers "B.Cu" "B.Paste" "B.Mask") (roundrect_rratio 0.25) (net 1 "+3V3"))
  (pad "2" smd roundrect (at 0.95 0 90) (size 1 1.45) (layers "B.Cu" "B.Paste" "B.Mask") (roundrect_rratio 0.25) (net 3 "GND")))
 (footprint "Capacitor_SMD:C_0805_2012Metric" (layer "B.Cu") (at 123 50)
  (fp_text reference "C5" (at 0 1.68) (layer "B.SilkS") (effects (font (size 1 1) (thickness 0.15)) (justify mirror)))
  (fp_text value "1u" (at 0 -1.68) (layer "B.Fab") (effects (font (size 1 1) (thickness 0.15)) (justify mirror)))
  (pad "1" smd roundrect (at -0.95 0) (size 1 1.45) (layers "B.Cu" "B.Paste" "B.Mask") (roundrect_rratio 0.25) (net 53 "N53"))
  (pad "2" smd roundrect (at 0.95 0) (size 1 1.45) (layers "B.Cu" "B.Paste" "B.Mask") (roundrect_rratio 0.25) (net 21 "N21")))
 (gr_line (start 30 25) (end 130 25) (layer "Edge.Cuts") (width 0.15))
 (gr_line (start 130 25) (end 130 75) (layer "Edge.Cuts") (width 0.15))
 (gr_line (start 30 75) (end 130 75) (layer "Edge.Cuts") (width 0.15))
 (gr_line (start 30 25) (end 30 75) (layer "Edge.Cuts") (width 0.15))
 (segment (start 64.175 48.5) (end 49.05 48.5) (width 0.3) (layer "F.Cu") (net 9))
 (segment (start 45.275 44.725) (end 44.575 44.025) (width 0.3) (layer "F.Cu") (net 9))
 (segment (start 44.575 44.025) (end 44.575 42.6) (width 0.3) (layer "F.Cu") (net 9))
 (segment (start 49.05 48.5) (end 45.275 44.725) (width 0.3) (layer "F.Cu") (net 9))
 (via (at 44.575 42.6) (size 0.8) (drill 0.4) (layers "F.Cu" "B.Cu") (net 9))
 (segment (start 44.575 42.6) (end 44.575 41.115) (width 0.3) (layer "B.Cu") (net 9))
 (segment (start 44.575 41.115) (end 44.57 41.11) (width 0.3) (layer "B.Cu") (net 9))
 (segment (start 64.175 49.3) (end 52.2 49.3) (width 0.3) (layer "F.Cu") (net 10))
 (via (at 52.2 49.3) (size 0.8) (drill 0.4) (layers "F.Cu" "B.Cu") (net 10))
 (segment (start 52.2 41.12) (end 52.19 41.11) (width 0.3) (layer "B.Cu") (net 10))
 (segment (start 52.2 49.3) (end 52.2 41.12) (width 0.3) (layer "B.Cu") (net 10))
 (segment (start 49.85 50.1) (end 64.175 50.1) (width 0.3) (layer "F.Cu") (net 11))
 (segment (start 44.675 44.925) (end 49.85 50.1) (width 0.3) (layer "F.Cu") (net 11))
 (segment (start 39.525 44.925) (end 44.675 44.925) (width 0.3) (layer "F.Cu") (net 11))
 (via (at 39.525 44.925) (size 0.8) (drill 0.4) (layers "F.Cu" "B.Cu") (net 11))
 (segment (start 39.525 41.145) (end 39.49 41.11) (width 0.3) (layer "B.Cu") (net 11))
 (segment (start 39.525 44.925) (end 39.525 41.145) (width 0.3) (layer "B.Cu") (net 11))
 (segment (start 49.825 50.9) (end 64.175 50.9) (width 0.3) (layer "F.Cu") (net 12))
 (segment (start 42.05 45.725) (end 44.65 45.725) (width 0.3) (layer "F.Cu") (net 12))
 (segment (start 44.65 45.725) (end 49.825 50.9) (width 0.3) (layer "F.Cu") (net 12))
 (via (at 42.05 45.725) (size 0.8) (drill 0.4) (layers "F.Cu" "B.Cu") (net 12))
 (segment (start 42.05 41.13) (end 42.03 41.11) (width 0.3) (layer "B.Cu") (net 12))
 (segment (start 42.05 45.725) (end 42.05 41.13) (width 0.3) (layer "B.Cu") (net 12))
 (segment (start 47.1 51.7) (end 64.175 51.7) (width 0.3) (layer "F.Cu") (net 13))
 (via (at 47.1 51.7) (size 0.8) (drill 0.4) (layers "F.Cu" "B.Cu") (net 13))
 (segment (start 47.1 41.12) (end 47.11 41.11) (width 0.3) (layer "B.Cu") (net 13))
 (segment (start 47.1 51.7) (end 47.1 41.12) (width 0.3) (layer "B.Cu") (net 13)))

